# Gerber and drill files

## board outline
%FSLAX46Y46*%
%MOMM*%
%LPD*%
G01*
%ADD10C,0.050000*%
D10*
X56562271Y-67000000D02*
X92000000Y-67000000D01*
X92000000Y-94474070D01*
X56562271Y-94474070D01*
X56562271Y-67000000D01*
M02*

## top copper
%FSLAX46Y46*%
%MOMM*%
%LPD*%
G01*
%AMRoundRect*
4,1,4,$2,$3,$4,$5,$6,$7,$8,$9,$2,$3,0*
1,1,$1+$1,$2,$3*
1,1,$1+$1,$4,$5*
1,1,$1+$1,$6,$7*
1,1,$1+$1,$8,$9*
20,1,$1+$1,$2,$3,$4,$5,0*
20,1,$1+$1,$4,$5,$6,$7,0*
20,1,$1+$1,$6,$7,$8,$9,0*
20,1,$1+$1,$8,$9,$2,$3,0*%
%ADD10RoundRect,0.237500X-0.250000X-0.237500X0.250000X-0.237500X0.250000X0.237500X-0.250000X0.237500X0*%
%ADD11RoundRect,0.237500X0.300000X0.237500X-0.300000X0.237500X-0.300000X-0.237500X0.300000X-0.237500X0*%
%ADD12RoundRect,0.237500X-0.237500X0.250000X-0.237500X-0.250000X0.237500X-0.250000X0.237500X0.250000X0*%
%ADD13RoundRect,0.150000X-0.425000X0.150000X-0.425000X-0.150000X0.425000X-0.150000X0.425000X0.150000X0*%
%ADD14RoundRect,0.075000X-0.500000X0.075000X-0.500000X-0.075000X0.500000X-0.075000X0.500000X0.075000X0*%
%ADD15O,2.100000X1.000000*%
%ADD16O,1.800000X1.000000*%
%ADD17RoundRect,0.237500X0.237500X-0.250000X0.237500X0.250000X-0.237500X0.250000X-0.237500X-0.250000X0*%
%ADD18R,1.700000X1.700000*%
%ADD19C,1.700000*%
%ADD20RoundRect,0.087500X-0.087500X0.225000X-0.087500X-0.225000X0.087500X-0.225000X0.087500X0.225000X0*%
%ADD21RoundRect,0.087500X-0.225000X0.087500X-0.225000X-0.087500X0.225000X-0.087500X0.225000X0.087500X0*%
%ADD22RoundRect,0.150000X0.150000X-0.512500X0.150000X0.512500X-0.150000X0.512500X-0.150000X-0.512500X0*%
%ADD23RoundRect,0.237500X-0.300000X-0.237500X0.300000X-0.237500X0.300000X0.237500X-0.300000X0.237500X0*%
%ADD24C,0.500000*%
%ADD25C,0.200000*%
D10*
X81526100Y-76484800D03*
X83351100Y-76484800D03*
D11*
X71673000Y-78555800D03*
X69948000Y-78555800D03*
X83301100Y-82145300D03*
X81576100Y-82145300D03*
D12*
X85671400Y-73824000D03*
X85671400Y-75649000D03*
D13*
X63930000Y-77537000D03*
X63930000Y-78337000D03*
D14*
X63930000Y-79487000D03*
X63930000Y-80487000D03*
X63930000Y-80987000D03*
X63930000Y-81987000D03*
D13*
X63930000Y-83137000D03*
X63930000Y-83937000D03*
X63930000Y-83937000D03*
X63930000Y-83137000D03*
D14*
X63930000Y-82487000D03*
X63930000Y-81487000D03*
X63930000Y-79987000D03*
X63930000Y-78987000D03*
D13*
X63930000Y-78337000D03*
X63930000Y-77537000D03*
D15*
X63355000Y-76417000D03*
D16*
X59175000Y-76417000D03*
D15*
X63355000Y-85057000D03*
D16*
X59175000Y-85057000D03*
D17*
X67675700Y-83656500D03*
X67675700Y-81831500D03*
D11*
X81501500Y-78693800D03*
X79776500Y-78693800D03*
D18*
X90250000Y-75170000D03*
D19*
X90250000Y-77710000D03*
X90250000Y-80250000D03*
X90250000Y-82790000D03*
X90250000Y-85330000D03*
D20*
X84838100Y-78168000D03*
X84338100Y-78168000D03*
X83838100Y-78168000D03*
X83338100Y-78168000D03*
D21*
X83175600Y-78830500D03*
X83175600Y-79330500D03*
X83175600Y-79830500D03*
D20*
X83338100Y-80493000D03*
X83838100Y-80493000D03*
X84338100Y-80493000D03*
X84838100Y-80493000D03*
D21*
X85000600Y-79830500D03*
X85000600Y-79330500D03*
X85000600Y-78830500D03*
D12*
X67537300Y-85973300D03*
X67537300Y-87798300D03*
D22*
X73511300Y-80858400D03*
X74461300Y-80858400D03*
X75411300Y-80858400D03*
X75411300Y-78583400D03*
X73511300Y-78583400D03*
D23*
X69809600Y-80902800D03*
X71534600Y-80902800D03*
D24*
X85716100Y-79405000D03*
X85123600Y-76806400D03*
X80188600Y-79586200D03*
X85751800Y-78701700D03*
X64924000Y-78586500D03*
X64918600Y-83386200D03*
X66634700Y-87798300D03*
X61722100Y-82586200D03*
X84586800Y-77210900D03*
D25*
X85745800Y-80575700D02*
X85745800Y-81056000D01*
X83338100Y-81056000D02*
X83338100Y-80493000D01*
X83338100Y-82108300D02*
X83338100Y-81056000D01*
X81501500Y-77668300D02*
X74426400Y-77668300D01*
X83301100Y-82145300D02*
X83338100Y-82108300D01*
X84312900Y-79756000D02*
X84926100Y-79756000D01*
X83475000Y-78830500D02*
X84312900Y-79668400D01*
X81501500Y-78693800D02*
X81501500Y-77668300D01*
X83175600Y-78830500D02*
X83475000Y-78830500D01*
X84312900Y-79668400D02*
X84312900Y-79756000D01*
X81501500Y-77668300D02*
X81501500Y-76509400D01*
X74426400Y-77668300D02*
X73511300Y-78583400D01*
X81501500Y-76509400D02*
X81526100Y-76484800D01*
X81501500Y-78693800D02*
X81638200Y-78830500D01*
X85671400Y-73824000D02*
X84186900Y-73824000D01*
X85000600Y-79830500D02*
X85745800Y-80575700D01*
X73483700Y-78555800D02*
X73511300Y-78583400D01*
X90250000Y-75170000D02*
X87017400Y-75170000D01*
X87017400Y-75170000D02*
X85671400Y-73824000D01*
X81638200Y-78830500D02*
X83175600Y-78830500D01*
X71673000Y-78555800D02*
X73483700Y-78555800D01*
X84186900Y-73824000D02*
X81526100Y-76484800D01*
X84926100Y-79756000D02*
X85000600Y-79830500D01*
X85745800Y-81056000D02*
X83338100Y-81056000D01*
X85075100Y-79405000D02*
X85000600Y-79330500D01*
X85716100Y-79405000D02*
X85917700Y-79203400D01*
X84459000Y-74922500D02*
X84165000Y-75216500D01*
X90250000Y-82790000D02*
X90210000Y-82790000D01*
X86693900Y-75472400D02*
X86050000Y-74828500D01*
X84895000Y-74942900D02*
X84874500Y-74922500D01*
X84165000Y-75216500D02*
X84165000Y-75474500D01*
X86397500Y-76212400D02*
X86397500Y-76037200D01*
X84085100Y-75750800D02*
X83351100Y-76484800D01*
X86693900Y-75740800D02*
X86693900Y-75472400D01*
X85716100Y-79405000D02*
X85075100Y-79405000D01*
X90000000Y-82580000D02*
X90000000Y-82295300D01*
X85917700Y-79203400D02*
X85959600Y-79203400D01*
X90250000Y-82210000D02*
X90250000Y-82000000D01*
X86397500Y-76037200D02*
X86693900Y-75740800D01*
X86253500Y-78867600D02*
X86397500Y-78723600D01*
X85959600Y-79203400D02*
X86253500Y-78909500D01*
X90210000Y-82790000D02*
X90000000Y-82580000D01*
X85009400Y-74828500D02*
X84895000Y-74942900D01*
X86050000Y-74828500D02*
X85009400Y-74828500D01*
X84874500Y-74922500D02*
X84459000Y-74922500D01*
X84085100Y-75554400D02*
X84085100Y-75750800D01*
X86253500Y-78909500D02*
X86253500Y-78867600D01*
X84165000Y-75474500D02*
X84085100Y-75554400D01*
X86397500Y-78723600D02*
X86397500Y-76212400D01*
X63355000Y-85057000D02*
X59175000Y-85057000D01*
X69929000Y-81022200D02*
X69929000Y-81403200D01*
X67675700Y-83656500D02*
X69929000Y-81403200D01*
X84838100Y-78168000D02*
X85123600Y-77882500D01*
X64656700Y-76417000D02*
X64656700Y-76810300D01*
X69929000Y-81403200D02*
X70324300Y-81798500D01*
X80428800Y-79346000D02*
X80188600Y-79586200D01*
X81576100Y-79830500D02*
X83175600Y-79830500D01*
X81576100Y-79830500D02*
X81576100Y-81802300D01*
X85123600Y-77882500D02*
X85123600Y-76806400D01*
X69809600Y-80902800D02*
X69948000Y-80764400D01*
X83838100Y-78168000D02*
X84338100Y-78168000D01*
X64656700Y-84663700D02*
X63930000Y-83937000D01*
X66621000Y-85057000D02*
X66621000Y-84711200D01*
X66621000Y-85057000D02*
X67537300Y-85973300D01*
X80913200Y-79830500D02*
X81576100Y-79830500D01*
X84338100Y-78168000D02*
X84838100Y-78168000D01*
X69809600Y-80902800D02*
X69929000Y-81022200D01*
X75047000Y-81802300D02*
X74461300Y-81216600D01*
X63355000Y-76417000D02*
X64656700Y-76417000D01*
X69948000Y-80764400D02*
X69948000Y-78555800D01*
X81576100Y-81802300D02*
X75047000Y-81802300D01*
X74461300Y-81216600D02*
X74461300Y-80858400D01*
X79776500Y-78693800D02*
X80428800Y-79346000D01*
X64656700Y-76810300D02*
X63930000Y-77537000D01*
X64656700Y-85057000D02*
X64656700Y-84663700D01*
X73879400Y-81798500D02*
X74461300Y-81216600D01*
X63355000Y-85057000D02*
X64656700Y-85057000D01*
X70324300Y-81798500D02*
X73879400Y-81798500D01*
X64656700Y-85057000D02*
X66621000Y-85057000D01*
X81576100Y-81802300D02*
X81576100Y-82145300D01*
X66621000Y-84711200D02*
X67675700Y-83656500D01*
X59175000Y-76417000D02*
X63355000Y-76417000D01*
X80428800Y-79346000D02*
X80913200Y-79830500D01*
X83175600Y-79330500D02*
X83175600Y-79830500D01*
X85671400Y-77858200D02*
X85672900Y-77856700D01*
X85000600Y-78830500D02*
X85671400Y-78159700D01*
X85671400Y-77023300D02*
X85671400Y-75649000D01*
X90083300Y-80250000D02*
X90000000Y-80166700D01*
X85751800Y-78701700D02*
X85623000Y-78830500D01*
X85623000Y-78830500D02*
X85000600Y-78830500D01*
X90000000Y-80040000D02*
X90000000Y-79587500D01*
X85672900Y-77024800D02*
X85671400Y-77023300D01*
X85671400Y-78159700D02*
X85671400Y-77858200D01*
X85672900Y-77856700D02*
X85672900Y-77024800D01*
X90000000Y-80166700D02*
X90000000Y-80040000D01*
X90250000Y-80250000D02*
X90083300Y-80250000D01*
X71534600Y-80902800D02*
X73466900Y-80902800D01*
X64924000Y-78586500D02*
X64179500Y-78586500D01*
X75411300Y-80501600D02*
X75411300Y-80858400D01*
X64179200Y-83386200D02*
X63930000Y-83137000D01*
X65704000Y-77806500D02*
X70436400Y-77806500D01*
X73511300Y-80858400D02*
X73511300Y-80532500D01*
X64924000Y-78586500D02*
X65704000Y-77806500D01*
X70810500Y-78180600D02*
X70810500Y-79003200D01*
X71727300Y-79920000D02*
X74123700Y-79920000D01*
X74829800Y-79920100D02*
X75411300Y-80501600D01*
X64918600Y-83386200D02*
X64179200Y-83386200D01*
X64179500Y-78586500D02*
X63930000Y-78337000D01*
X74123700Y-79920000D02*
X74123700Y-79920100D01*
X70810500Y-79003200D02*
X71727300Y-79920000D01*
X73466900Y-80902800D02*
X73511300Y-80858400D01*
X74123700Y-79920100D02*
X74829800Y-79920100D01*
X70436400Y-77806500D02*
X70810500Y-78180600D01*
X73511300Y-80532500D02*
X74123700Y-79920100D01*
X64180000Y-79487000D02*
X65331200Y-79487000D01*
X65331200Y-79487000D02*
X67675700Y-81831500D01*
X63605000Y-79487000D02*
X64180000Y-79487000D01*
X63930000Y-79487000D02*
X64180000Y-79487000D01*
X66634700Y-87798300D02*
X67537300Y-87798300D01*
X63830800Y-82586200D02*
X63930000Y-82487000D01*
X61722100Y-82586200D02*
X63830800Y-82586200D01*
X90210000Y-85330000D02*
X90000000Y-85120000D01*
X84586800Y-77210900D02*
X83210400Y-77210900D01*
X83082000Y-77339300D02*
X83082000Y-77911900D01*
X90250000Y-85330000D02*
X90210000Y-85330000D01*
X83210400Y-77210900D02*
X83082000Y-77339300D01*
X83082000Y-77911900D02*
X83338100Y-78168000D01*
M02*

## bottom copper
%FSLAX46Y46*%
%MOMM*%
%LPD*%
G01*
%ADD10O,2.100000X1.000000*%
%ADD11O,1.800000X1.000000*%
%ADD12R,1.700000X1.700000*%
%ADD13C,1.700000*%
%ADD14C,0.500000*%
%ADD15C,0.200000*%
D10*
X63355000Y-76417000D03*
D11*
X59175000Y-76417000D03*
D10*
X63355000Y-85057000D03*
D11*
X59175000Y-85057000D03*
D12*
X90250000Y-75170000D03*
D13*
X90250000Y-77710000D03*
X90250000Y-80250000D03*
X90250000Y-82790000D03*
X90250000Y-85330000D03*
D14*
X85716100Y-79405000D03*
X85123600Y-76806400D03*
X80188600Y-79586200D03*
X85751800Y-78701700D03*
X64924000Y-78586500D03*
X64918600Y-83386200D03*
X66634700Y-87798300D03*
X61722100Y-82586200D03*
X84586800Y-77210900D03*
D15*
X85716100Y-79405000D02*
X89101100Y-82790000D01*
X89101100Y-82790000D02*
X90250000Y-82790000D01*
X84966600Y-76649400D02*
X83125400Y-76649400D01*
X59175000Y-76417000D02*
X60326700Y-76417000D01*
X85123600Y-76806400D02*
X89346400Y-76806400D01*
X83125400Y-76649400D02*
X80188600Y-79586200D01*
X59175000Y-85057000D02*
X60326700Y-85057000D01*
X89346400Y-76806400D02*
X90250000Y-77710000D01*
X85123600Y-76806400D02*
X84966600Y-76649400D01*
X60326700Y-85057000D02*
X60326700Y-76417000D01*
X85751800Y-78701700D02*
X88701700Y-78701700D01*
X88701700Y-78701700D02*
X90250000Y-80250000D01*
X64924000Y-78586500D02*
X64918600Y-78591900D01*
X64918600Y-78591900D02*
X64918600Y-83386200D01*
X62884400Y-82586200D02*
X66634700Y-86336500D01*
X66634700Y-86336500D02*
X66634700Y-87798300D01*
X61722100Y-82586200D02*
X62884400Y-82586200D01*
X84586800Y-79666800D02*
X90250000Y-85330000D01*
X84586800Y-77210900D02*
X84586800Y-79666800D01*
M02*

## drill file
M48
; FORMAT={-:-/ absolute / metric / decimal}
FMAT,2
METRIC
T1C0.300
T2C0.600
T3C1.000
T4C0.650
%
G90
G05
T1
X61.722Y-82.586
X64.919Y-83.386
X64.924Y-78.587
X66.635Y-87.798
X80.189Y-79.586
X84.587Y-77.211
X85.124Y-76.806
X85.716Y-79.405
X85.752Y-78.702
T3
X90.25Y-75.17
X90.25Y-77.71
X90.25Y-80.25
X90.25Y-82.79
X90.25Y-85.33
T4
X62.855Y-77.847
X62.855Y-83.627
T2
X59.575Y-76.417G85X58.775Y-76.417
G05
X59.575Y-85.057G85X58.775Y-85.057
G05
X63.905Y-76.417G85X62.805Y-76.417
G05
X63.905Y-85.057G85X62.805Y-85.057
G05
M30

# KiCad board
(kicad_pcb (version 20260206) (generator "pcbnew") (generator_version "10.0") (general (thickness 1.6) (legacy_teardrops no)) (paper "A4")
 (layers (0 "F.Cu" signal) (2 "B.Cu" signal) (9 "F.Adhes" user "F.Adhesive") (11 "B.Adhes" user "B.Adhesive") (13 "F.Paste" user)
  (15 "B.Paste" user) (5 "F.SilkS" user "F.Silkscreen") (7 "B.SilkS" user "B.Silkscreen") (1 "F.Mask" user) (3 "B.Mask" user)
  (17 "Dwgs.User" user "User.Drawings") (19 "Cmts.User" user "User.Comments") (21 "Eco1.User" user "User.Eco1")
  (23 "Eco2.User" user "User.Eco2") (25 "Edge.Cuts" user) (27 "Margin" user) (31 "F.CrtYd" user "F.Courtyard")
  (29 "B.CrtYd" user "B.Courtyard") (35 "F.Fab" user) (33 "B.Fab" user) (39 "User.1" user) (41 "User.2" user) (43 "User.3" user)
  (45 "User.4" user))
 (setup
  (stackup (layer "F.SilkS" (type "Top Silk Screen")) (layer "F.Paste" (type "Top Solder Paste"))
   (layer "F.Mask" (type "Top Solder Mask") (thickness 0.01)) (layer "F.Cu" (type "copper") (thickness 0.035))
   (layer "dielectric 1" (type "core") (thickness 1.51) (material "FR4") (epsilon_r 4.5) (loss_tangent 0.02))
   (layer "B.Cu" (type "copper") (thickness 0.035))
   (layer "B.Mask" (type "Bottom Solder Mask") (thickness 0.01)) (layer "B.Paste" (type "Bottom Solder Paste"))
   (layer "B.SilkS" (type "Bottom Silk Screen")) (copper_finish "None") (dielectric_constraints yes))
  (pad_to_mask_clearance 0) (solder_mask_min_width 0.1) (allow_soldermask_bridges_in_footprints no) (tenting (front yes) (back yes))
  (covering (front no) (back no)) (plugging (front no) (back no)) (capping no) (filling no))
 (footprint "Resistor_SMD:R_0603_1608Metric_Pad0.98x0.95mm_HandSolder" (layer "F.Cu") (at 82.4386 76.4848)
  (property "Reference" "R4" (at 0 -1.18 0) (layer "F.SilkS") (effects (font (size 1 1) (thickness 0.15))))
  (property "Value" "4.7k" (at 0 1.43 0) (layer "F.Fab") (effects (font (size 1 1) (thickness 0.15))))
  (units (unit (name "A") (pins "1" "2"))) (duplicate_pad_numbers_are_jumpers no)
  (pad "1" smd roundrect (at -0.9125 0) (size 0.975 0.95) (layers "F.Cu" "F.Mask" "F.Paste") (roundrect_rratio 0.25) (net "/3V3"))
  (pad "2" smd roundrect (at 0.9125 0) (size 0.975 0.95) (layers "F.Cu" "F.Mask" "F.Paste") (roundrect_rratio 0.25) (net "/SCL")))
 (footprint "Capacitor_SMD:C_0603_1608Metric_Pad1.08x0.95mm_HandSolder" (layer "F.Cu") (at 70.8105 78.5558 180)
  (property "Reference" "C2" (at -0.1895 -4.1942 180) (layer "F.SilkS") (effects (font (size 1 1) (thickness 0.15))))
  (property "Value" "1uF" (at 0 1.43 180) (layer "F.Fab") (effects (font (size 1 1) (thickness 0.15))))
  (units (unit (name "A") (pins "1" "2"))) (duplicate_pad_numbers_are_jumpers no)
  (pad "1" smd roundrect (at -0.8625 0 180) (size 1.075 0.95) (layers "F.Cu" "F.Mask" "F.Paste") (roundrect_rratio 0.25) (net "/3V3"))
  (pad "2" smd roundrect (at 0.8625 0 180) (size 1.075 0.95) (layers "F.Cu" "F.Mask" "F.Paste") (roundrect_rratio 0.25) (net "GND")))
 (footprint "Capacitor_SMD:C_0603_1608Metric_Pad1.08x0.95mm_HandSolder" (layer "F.Cu") (at 82.4386 82.1453 180)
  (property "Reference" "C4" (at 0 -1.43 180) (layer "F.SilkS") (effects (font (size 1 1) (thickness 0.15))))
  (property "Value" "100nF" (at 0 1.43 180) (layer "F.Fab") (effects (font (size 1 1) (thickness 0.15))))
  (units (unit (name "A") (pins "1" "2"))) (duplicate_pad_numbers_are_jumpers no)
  (pad "1" smd roundrect (at -0.8625 0 180) (size 1.075 0.95) (layers "F.Cu" "F.Mask" "F.Paste") (roundrect_rratio 0.25) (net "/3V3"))
  (pad "2" smd roundrect (at 0.8625 0 180) (size 1.075 0.95) (layers "F.Cu" "F.Mask" "F.Paste") (roundrect_rratio 0.25) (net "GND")))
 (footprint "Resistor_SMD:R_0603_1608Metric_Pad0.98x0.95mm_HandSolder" (layer "F.Cu") (at 85.6714 74.7365 -90)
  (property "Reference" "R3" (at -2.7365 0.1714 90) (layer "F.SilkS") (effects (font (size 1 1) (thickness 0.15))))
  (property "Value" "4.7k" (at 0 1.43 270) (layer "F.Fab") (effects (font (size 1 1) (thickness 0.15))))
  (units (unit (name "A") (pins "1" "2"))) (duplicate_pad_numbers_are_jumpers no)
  (pad "1" smd roundrect (at -0.9125 0 270) (size 0.975 0.95) (layers "F.Cu" "F.Mask" "F.Paste") (roundrect_rratio 0.25) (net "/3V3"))
  (pad "2" smd roundrect (at 0.9125 0 270) (size 0.975 0.95) (layers "F.Cu" "F.Mask" "F.Paste") (roundrect_rratio 0.25) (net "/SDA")))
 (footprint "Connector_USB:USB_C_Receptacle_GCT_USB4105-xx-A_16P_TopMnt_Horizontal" (layer "F.Cu") (at 60.25 80.737 -90)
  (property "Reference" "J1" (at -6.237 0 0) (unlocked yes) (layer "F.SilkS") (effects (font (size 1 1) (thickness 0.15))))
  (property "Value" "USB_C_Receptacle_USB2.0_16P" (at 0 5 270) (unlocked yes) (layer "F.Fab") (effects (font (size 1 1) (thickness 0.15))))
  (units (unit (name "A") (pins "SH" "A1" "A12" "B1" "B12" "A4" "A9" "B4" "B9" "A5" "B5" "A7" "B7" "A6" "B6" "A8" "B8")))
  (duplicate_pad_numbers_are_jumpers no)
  (pad "" np_thru_hole circle (at -2.89 -2.605 270) (size 0.65 0.65) (drill 0.65) (layers "*.Cu" "*.Mask"))
  (pad "" np_thru_hole circle (at 2.89 -2.605 270) (size 0.65 0.65) (drill 0.65) (layers "*.Cu" "*.Mask"))
  (pad "A1" smd roundrect (at -3.2 -3.68 270) (size 0.6 1.15) (layers "F.Cu" "F.Mask" "F.Paste") (roundrect_rratio 0.25) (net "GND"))
  (pad "A4" smd roundrect (at -2.4 -3.68 270) (size 0.6 1.15) (layers "F.Cu" "F.Mask" "F.Paste") (roundrect_rratio 0.25) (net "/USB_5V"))
  (pad "A5" smd roundrect (at -1.25 -3.68 270) (size 0.3 1.15) (layers "F.Cu" "F.Mask" "F.Paste") (roundrect_rratio 0.25)
   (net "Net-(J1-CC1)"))
  (pad "A6" smd roundrect (at -0.25 -3.68 270) (size 0.3 1.15) (layers "F.Cu" "F.Mask" "F.Paste") (roundrect_rratio 0.25)
   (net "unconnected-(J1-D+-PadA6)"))
  (pad "A7" smd roundrect (at 0.25 -3.68 270) (size 0.3 1.15) (layers "F.Cu" "F.Mask" "F.Paste") (roundrect_rratio 0.25)
   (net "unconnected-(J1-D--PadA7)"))
  (pad "A8" smd roundrect (at 1.25 -3.68 270) (size 0.3 1.15) (layers "F.Cu" "F.Mask" "F.Paste") (roundrect_rratio 0.25)
   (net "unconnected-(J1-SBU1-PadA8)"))
  (pad "A9" smd roundrect (at 2.4 -3.68 270) (size 0.6 1.15) (layers "F.Cu" "F.Mask" "F.Paste") (roundrect_rratio 0.25) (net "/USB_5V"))
  (pad "A12" smd roundrect (at 3.2 -3.68 270) (size 0.6 1.15) (layers "F.Cu" "F.Mask" "F.Paste") (roundrect_rratio 0.25) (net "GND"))
  (pad "B1" smd roundrect (at 3.2 -3.68 270) (size 0.6 1.15) (layers "F.Cu" "F.Mask" "F.Paste") (roundrect_rratio 0.25) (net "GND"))
  (pad "B4" smd roundrect (at 2.4 -3.68 270) (size 0.6 1.15) (layers "F.Cu" "F.Mask" "F.Paste") (roundrect_rratio 0.25) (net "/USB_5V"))
  (pad "B5" smd roundrect (at 1.75 -3.68 270) (size 0.3 1.15) (layers "F.Cu" "F.Mask" "F.Paste") (roundrect_rratio 0.25)
   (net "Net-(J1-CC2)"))
  (pad "B6" smd roundrect (at 0.75 -3.68 270) (size 0.3 1.15) (layers "F.Cu" "F.Mask" "F.Paste") (roundrect_rratio 0.25)
   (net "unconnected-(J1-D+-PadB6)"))
  (pad "B7" smd roundrect (at -0.75 -3.68 270) (size 0.3 1.15) (layers "F.Cu" "F.Mask" "F.Paste") (roundrect_rratio 0.25)
   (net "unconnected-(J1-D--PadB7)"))
  (pad "B8" smd roundrect (at -1.75 -3.68 270) (size 0.3 1.15) (layers "F.Cu" "F.Mask" "F.Paste") (roundrect_rratio 0.25)
   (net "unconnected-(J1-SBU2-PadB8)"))
  (pad "B9" smd roundrect (at -2.4 -3.68 270) (size 0.6 1.15) (layers "F.Cu" "F.Mask" "F.Paste") (roundrect_rratio 0.25) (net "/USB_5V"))
  (pad "B12" smd roundrect (at -3.2 -3.68 270) (size 0.6 1.15) (layers "F.Cu" "F.Mask" "F.Paste") (roundrect_rratio 0.25) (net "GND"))
  (pad "SH" thru_hole oval (at -4.32 -3.105 270) (size 1 2.1) (drill oval 0.6 1.7) (layers "*.Cu" "*.Mask" "F.Paste")
   (remove_unused_layers no) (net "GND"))
  (pad "SH" thru_hole oval (at -4.32 1.075 270) (size 1 1.8) (drill oval 0.6 1.4) (layers "*.Cu" "*.Mask" "F.Paste")
   (remove_unused_layers no) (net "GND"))
  (pad "SH" thru_hole oval (at 4.32 -3.105 270) (size 1 2.1) (drill oval 0.6 1.7) (layers "*.Cu" "*.Mask" "F.Paste")
   (remove_unused_layers no) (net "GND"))
  (pad "SH" thru_hole oval (at 4.32 1.075 270) (size 1 1.8) (drill oval 0.6 1.4) (layers "*.Cu" "*.Mask" "F.Paste")
   (remove_unused_layers no) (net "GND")))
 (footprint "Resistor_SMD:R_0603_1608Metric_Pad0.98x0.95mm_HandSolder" (layer "F.Cu") (at 67.6757 82.744 90)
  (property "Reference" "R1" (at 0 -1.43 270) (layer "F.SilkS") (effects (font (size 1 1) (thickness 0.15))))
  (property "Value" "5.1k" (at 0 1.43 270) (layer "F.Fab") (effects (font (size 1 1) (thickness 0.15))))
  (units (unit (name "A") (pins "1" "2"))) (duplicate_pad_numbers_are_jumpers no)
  (pad "1" smd roundrect (at -0.9125 0 90) (size 0.975 0.95) (layers "F.Cu" "F.Mask" "F.Paste") (roundrect_rratio 0.25) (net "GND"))
  (pad "2" smd roundrect (at 0.9125 0 90) (size 0.975 0.95) (layers "F.Cu" "F.Mask" "F.Paste") (roundrect_rratio 0.25) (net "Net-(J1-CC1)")))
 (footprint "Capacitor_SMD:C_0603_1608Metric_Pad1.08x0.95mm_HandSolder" (layer "F.Cu") (at 80.639 78.6938 180)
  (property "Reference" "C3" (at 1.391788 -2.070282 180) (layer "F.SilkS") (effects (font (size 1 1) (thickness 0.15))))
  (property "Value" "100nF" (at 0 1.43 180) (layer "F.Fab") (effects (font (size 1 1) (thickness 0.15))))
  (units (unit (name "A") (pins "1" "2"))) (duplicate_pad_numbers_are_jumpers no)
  (pad "1" smd roundrect (at -0.8625 0 180) (size 1.075 0.95) (layers "F.Cu" "F.Mask" "F.Paste") (roundrect_rratio 0.25) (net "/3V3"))
  (pad "2" smd roundrect (at 0.8625 0 180) (size 1.075 0.95) (layers "F.Cu" "F.Mask" "F.Paste") (roundrect_rratio 0.25) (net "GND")))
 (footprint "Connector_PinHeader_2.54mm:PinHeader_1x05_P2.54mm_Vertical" (layer "F.Cu") (at 90.25 75.17)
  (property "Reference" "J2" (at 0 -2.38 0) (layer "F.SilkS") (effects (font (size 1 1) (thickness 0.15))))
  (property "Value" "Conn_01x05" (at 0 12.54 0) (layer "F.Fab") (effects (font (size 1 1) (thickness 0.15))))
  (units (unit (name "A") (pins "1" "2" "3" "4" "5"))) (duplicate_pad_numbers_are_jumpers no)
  (pad "1" thru_hole rect (at 0 0) (size 1.7 1.7) (drill 1) (layers "*.Cu" "*.Mask") (remove_unused_layers no) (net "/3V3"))
  (pad "2" thru_hole circle (at 0 2.54) (size 1.7 1.7) (drill 1) (layers "*.Cu" "*.Mask") (remove_unused_layers no) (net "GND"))
  (pad "3" thru_hole circle (at 0 5.08) (size 1.7 1.7) (drill 1) (layers "*.Cu" "*.Mask") (remove_unused_layers no) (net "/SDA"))
  (pad "4" thru_hole circle (at 0 7.62) (size 1.7 1.7) (drill 1) (layers "*.Cu" "*.Mask") (remove_unused_layers no) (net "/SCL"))
  (pad "5" thru_hole circle (at 0 10.16) (size 1.7 1.7) (drill 1) (layers "*.Cu" "*.Mask") (remove_unused_layers no) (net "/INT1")))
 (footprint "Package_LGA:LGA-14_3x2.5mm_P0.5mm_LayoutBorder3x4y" (layer "F.Cu") (at 84.0881 79.3305 -90)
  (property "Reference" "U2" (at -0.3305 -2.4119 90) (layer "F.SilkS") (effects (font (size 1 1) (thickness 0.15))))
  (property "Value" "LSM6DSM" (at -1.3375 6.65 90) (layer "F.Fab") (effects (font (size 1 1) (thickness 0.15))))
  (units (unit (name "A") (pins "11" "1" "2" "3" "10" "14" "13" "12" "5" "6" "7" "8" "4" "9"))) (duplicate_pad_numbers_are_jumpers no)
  (pad "1" smd roundrect (at -1.1625 -0.75 270) (size 0.625 0.35) (layers "F.Cu" "F.Mask" "F.Paste") (roundrect_rratio 0.25) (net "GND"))
  (pad "2" smd roundrect (at -1.1625 -0.25 270) (size 0.625 0.35) (layers "F.Cu" "F.Mask" "F.Paste") (roundrect_rratio 0.25) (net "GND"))
  (pad "3" smd roundrect (at -1.1625 0.25 270) (size 0.625 0.35) (layers "F.Cu" "F.Mask" "F.Paste") (roundrect_rratio 0.25) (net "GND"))
  (pad "4" smd roundrect (at -1.1625 0.75 270) (size 0.625 0.35) (layers "F.Cu" "F.Mask" "F.Paste") (roundrect_rratio 0.25) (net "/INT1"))
  (pad "5" smd roundrect (at -0.5 0.9125 270) (size 0.35 0.625) (layers "F.Cu" "F.Mask" "F.Paste") (roundrect_rratio 0.25) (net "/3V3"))
  (pad "6" smd roundrect (at 0 0.9125 270) (size 0.35 0.625) (layers "F.Cu" "F.Mask" "F.Paste") (roundrect_rratio 0.25) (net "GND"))
  (pad "7" smd roundrect (at 0.5 0.9125 270) (size 0.35 0.625) (layers "F.Cu" "F.Mask" "F.Paste") (roundrect_rratio 0.25) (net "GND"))
  (pad "8" smd roundrect (at 1.1625 0.75 270) (size 0.625 0.35) (layers "F.Cu" "F.Mask" "F.Paste") (roundrect_rratio 0.25) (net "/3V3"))
  (pad "9" smd roundrect (at 1.1625 0.25 270) (size 0.625 0.35) (layers "F.Cu" "F.Mask" "F.Paste") (roundrect_rratio 0.25)
   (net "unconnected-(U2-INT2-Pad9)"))
  (pad "10" smd roundrect (at 1.1625 -0.25 270) (size 0.625 0.35) (layers "F.Cu" "F.Mask" "F.Paste") (roundrect_rratio 0.25)
   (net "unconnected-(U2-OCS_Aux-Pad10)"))
  (pad "11" smd roundrect (at 1.1625 -0.75 270) (size 0.625 0.35) (layers "F.Cu" "F.Mask" "F.Paste") (roundrect_rratio 0.25)
   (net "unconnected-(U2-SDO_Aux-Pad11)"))
  (pad "12" smd roundrect (at 0.5 -0.9125 270) (size 0.35 0.625) (layers "F.Cu" "F.Mask" "F.Paste") (roundrect_rratio 0.25) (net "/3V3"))
  (pad "13" smd roundrect (at 0 -0.9125 270) (size 0.35 0.625) (layers "F.Cu" "F.Mask" "F.Paste") (roundrect_rratio 0.25) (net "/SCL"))
  (pad "14" smd roundrect (at -0.5 -0.9125 270) (size 0.35 0.625) (layers "F.Cu" "F.Mask" "F.Paste") (roundrect_rratio 0.25) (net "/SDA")))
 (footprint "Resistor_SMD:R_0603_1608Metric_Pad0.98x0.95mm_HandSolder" (layer "F.Cu") (at 67.5373 86.8858 -90)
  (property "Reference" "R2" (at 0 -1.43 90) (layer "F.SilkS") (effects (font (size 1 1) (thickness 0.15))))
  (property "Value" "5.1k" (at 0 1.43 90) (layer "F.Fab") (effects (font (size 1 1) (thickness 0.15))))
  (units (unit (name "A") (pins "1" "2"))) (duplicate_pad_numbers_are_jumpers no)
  (pad "1" smd roundrect (at -0.9125 0 270) (size 0.975 0.95) (layers "F.Cu" "F.Mask" "F.Paste") (roundrect_rratio 0.25) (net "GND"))
  (pad "2" smd roundrect (at 0.9125 0 270) (size 0.975 0.95) (layers "F.Cu" "F.Mask" "F.Paste") (roundrect_rratio 0.25) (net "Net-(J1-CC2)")))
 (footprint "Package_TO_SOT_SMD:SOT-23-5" (layer "F.Cu") (at 74.4613 79.7209 90)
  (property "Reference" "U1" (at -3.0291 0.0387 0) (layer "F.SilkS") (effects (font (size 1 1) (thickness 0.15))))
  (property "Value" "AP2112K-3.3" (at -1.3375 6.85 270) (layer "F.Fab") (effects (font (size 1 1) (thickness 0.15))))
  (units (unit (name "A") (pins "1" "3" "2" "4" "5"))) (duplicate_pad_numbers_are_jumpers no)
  (pad "1" smd roundrect (at -1.1375 -0.95 90) (size 1.325 0.6) (layers "F.Cu" "F.Mask" "F.Paste") (roundrect_rratio 0.25) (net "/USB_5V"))
  (pad "2" smd roundrect (at -1.1375 0 90) (size 1.325 0.6) (layers "F.Cu" "F.Mask" "F.Paste") (roundrect_rratio 0.25) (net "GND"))
  (pad "3" smd roundrect (at -1.1375 0.95 90) (size 1.325 0.6) (layers "F.Cu" "F.Mask" "F.Paste") (roundrect_rratio 0.25) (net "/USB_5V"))
  (pad "4" smd roundrect (at 1.1375 0.95 90) (size 1.325 0.6) (layers "F.Cu" "F.Mask" "F.Paste") (roundrect_rratio 0.25)
   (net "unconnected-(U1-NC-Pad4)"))
  (pad "5" smd roundrect (at 1.1375 -0.95 90) (size 1.325 0.6) (layers "F.Cu" "F.Mask" "F.Paste") (roundrect_rratio 0.25) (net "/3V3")))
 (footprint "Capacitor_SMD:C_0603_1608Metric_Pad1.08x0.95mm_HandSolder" (layer "F.Cu") (at 70.6721 80.9028)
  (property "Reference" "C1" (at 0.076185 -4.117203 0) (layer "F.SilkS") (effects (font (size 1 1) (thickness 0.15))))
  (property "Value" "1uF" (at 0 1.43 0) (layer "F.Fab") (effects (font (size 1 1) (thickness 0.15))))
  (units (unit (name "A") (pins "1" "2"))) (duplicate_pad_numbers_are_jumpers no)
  (pad "1" smd roundrect (at -0.8625 0) (size 1.075 0.95) (layers "F.Cu" "F.Mask" "F.Paste") (roundrect_rratio 0.25) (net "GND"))
  (pad "2" smd roundrect (at 0.8625 0) (size 1.075 0.95) (layers "F.Cu" "F.Mask" "F.Paste") (roundrect_rratio 0.25) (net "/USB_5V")))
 (gr_rect (start 56.562271 67) (end 92 94.47407) (stroke (width 0.05) (type default)) (fill no) (layer "Edge.Cuts"))
 (segment (start 85.7458 80.5757) (end 85.7458 81.056) (width 0.2) (layer "F.Cu") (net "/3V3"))
 (segment (start 83.3381 81.056) (end 83.3381 80.493) (width 0.2) (layer "F.Cu") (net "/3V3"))
 (segment (start 83.3381 82.1083) (end 83.3381 81.056) (width 0.2) (layer "F.Cu") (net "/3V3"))
 (segment (start 81.5015 77.6683) (end 74.4264 77.6683) (width 0.2) (layer "F.Cu") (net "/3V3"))
 (segment (start 83.3011 82.1453) (end 83.3381 82.1083) (width 0.2) (layer "F.Cu") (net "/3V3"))
 (segment (start 84.3129 79.756) (end 84.9261 79.756) (width 0.2) (layer "F.Cu") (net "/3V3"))
 (segment (start 83.475 78.8305) (end 84.3129 79.6684) (width 0.2) (layer "F.Cu") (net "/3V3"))
 (segment (start 81.5015 78.6938) (end 81.5015 77.6683) (width 0.2) (layer "F.Cu") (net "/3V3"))
 (segment (start 83.1756 78.8305) (end 83.475 78.8305) (width 0.2) (layer "F.Cu") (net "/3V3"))
 (segment (start 84.3129 79.6684) (end 84.3129 79.756) (width 0.2) (layer "F.Cu") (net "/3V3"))
 (segment (start 81.5015 77.6683) (end 81.5015 76.5094) (width 0.2) (layer "F.Cu") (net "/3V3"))
 (segment (start 74.4264 77.6683) (end 73.5113 78.5834) (width 0.2) (layer "F.Cu") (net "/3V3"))
 (segment (start 81.5015 76.5094) (end 81.5261 76.4848) (width 0.2) (layer "F.Cu") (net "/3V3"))
 (segment (start 81.5015 78.6938) (end 81.6382 78.8305) (width 0.2) (layer "F.Cu") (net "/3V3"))
 (segment (start 85.6714 73.824) (end 84.1869 73.824) (width 0.2) (layer "F.Cu") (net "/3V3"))
 (segment (start 85.0006 79.8305) (end 85.7458 80.5757) (width 0.2) (layer "F.Cu") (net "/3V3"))
 (segment (start 73.4837 78.5558) (end 73.5113 78.5834) (width 0.2) (layer "F.Cu") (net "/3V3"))
 (segment (start 90.25 75.17) (end 87.0174 75.17) (width 0.2) (layer "F.Cu") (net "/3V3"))
 (segment (start 87.0174 75.17) (end 85.6714 73.824) (width 0.2) (layer "F.Cu") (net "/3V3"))
 (segment (start 81.6382 78.8305) (end 83.1756 78.8305) (width 0.2) (layer "F.Cu") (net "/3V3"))
 (segment (start 71.673 78.5558) (end 73.4837 78.5558) (width 0.2) (layer "F.Cu") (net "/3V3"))
 (segment (start 84.1869 73.824) (end 81.5261 76.4848) (width 0.2) (layer "F.Cu") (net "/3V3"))
 (segment (start 84.9261 79.756) (end 85.0006 79.8305) (width 0.2) (layer "F.Cu") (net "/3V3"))
 (segment (start 85.7458 81.056) (end 83.3381 81.056) (width 0.2) (layer "F.Cu") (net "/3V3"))
 (segment (start 85.0751 79.405) (end 85.0006 79.3305) (width 0.2) (layer "F.Cu") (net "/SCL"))
 (segment (start 85.7161 79.405) (end 85.9177 79.2034) (width 0.2) (layer "F.Cu") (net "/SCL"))
 (segment (start 84.459 74.9225) (end 84.165 75.2165) (width 0.2) (layer "F.Cu") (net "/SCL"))
 (segment (start 90.25 82.79) (end 90.21 82.79) (width 0.2) (layer "F.Cu") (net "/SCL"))
 (segment (start 86.6939 75.4724) (end 86.05 74.8285) (width 0.2) (layer "F.Cu") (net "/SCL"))
 (segment (start 84.895 74.9429) (end 84.8745 74.9225) (width 0.2) (layer "F.Cu") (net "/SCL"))
 (segment (start 84.165 75.2165) (end 84.165 75.4745) (width 0.2) (layer "F.Cu") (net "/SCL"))
 (segment (start 86.3975 76.2124) (end 86.3975 76.0372) (width 0.2) (layer "F.Cu") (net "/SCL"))
 (segment (start 84.0851 75.7508) (end 83.3511 76.4848) (width 0.2) (layer "F.Cu") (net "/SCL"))
 (segment (start 86.6939 75.7408) (end 86.6939 75.4724) (width 0.2) (layer "F.Cu") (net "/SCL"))
 (segment (start 85.7161 79.405) (end 85.0751 79.405) (width 0.2) (layer "F.Cu") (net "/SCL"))
 (segment (start 90 82.58) (end 90 82.2953) (width 0.2) (layer "F.Cu") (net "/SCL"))
 (segment (start 85.9177 79.2034) (end 85.9596 79.2034) (width 0.2) (layer "F.Cu") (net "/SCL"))
 (segment (start 90.25 82.21) (end 90.25 82) (width 0.2) (layer "F.Cu") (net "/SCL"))
 (segment (start 86.3975 76.0372) (end 86.6939 75.7408) (width 0.2) (layer "F.Cu") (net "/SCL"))
 (segment (start 86.2535 78.8676) (end 86.3975 78.7236) (width 0.2) (layer "F.Cu") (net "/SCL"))
 (segment (start 85.9596 79.2034) (end 86.2535 78.9095) (width 0.2) (layer "F.Cu") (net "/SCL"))
 (segment (start 90.21 82.79) (end 90 82.58) (width 0.2) (layer "F.Cu") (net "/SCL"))
 (segment (start 85.0094 74.8285) (end 84.895 74.9429) (width 0.2) (layer "F.Cu") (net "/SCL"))
 (segment (start 86.05 74.8285) (end 85.0094 74.8285) (width 0.2) (layer "F.Cu") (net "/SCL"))
 (segment (start 84.8745 74.9225) (end 84.459 74.9225) (width 0.2) (layer "F.Cu") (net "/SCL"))
 (segment (start 84.0851 75.5544) (end 84.0851 75.7508) (width 0.2) (layer "F.Cu") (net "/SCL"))
 (segment (start 86.2535 78.9095) (end 86.2535 78.8676) (width 0.2) (layer "F.Cu") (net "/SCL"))
 (segment (start 84.165 75.4745) (end 84.0851 75.5544) (width 0.2) (layer "F.Cu") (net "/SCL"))
 (segment (start 86.3975 78.7236) (end 86.3975 76.2124) (width 0.2) (layer "F.Cu") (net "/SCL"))
 (via (at 85.7161 79.405) (size 0.5) (drill 0.3) (layers "F.Cu" "B.Cu") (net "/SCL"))
 (segment (start 85.7161 79.405) (end 89.1011 82.79) (width 0.2) (layer "B.Cu") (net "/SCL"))
 (segment (start 89.1011 82.79) (end 90.25 82.79) (width 0.2) (layer "B.Cu") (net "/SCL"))
 (segment (start 63.355 85.057) (end 59.175 85.057) (width 0.2) (layer "F.Cu") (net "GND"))
 (segment (start 69.929 81.0222) (end 69.929 81.4032) (width 0.2) (layer "F.Cu") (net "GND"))
 (segment (start 67.6757 83.6565) (end 69.929 81.4032) (width 0.2) (layer "F.Cu") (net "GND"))
 (segment (start 84.8381 78.168) (end 85.1236 77.8825) (width 0.2) (layer "F.Cu") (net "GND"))
 (segment (start 64.6567 76.417) (end 64.6567 76.8103) (width 0.2) (layer "F.Cu") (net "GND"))
 (segment (start 69.929 81.4032) (end 70.3243 81.7985) (width 0.2) (layer "F.Cu") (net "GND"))
 (segment (start 80.4288 79.346) (end 80.1886 79.5862) (width 0.2) (layer "F.Cu") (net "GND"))
 (segment (start 81.5761 79.8305) (end 83.1756 79.8305) (width 0.2) (layer "F.Cu") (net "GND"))
 (segment (start 81.5761 79.8305) (end 81.5761 81.8023) (width 0.2) (layer "F.Cu") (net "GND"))
 (segment (start 85.1236 77.8825) (end 85.1236 76.8064) (width 0.2) (layer "F.Cu") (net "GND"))
 (segment (start 69.8096 80.9028) (end 69.948 80.7644) (width 0.2) (layer "F.Cu") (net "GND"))
 (segment (start 83.8381 78.168) (end 84.3381 78.168) (width 0.2) (layer "F.Cu") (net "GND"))
 (segment (start 64.6567 84.6637) (end 63.93 83.937) (width 0.2) (layer "F.Cu") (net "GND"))
 (segment (start 66.621 85.057) (end 66.621 84.7112) (width 0.2) (layer "F.Cu") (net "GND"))
 (segment (start 66.621 85.057) (end 67.5373 85.9733) (width 0.2) (layer "F.Cu") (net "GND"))
 (segment (start 80.9132 79.8305) (end 81.5761 79.8305) (width 0.2) (layer "F.Cu") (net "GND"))
 (segment (start 84.3381 78.168) (end 84.8381 78.168) (width 0.2) (layer "F.Cu") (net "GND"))
 (segment (start 69.8096 80.9028) (end 69.929 81.0222) (width 0.2) (layer "F.Cu") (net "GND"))
 (segment (start 75.047 81.8023) (end 74.4613 81.2166) (width 0.2) (layer "F.Cu") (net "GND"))
 (segment (start 63.355 76.417) (end 64.6567 76.417) (width 0.2) (layer "F.Cu") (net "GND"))
 (segment (start 69.948 80.7644) (end 69.948 78.5558) (width 0.2) (layer "F.Cu") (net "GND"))
 (segment (start 81.5761 81.8023) (end 75.047 81.8023) (width 0.2) (layer "F.Cu") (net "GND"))
 (segment (start 74.4613 81.2166) (end 74.4613 80.8584) (width 0.2) (layer "F.Cu") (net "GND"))
 (segment (start 79.7765 78.6938) (end 80.4288 79.346) (width 0.2) (layer "F.Cu") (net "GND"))
 (segment (start 64.6567 76.8103) (end 63.93 77.537) (width 0.2) (layer "F.Cu") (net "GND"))
 (segment (start 64.6567 85.057) (end 64.6567 84.6637) (width 0.2) (layer "F.Cu") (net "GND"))
 (segment (start 73.8794 81.7985) (end 74.4613 81.2166) (width 0.2) (layer "F.Cu") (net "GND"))
 (segment (start 63.355 85.057) (end 64.6567 85.057) (width 0.2) (layer "F.Cu") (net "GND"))
 (segment (start 70.3243 81.7985) (end 73.8794 81.7985) (width 0.2) (layer "F.Cu") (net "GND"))
 (segment (start 64.6567 85.057) (end 66.621 85.057) (width 0.2) (layer "F.Cu") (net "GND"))
 (segment (start 81.5761 81.8023) (end 81.5761 82.1453) (width 0.2) (layer "F.Cu") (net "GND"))
 (segment (start 66.621 84.7112) (end 67.6757 83.6565) (width 0.2) (layer "F.Cu") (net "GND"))
 (segment (start 59.175 76.417) (end 63.355 76.417) (width 0.2) (layer "F.Cu") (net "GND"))
 (segment (start 80.4288 79.346) (end 80.9132 79.8305) (width 0.2) (layer "F.Cu") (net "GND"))
 (segment (start 83.1756 79.3305) (end 83.1756 79.8305) (width 0.2) (layer "F.Cu") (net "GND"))
 (via (at 85.1236 76.8064) (size 0.5) (drill 0.3) (layers "F.Cu" "B.Cu") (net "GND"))
 (via (at 80.1886 79.5862) (size 0.5) (drill 0.3) (layers "F.Cu" "B.Cu") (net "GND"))
 (segment (start 84.9666 76.6494) (end 83.1254 76.6494) (width 0.2) (layer "B.Cu") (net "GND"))
 (segment (start 59.175 76.417) (end 60.3267 76.417) (width 0.2) (layer "B.Cu") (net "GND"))
 (segment (start 85.1236 76.8064) (end 89.3464 76.8064) (width 0.2) (layer "B.Cu") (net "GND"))
 (segment (start 83.1254 76.6494) (end 80.1886 79.5862) (width 0.2) (layer "B.Cu") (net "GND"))
 (segment (start 59.175 85.057) (end 60.3267 85.057) (width 0.2) (layer "B.Cu") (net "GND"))
 (segment (start 89.3464 76.8064) (end 90.25 77.71) (width 0.2) (layer "B.Cu") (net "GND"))
 (segment (start 85.1236 76.8064) (end 84.9666 76.6494) (width 0.2) (layer "B.Cu") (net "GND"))
 (segment (start 60.3267 85.057) (end 60.3267 76.417) (width 0.2) (layer "B.Cu") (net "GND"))
 (segment (start 85.6714 77.8582) (end 85.6729 77.8567) (width 0.2) (layer "F.Cu") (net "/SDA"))
 (segment (start 85.0006 78.8305) (end 85.6714 78.1597) (width 0.2) (layer "F.Cu") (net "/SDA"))
 (segment (start 85.6714 77.0233) (end 85.6714 75.649) (width 0.2) (layer "F.Cu") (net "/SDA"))
 (segment (start 90.0833 80.25) (end 90 80.1667) (width 0.2) (layer "F.Cu") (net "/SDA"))
 (segment (start 85.7518 78.7017) (end 85.623 78.8305) (width 0.2) (layer "F.Cu") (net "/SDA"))
 (segment (start 85.623 78.8305) (end 85.0006 78.8305) (width 0.2) (layer "F.Cu") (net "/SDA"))
 (segment (start 90 80.04) (end 90 79.5875) (width 0.2) (layer "F.Cu") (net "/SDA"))
 (segment (start 85.6729 77.0248) (end 85.6714 77.0233) (width 0.2) (layer "F.Cu") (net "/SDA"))
 (segment (start 85.6714 78.1597) (end 85.6714 77.8582) (width 0.2) (layer "F.Cu") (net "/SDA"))
 (segment (start 85.6729 77.8567) (end 85.6729 77.0248) (width 0.2) (layer "F.Cu") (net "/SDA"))
 (segment (start 90 80.1667) (end 90 80.04) (width 0.2) (layer "F.Cu") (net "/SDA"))
 (segment (start 90.25 80.25) (end 90.0833 80.25) (width 0.2) (layer "F.Cu") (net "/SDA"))
 (via (at 85.7518 78.7017) (size 0.5) (drill 0.3) (layers "F.Cu" "B.Cu") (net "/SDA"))
 (segment (start 85.7518 78.7017) (end 88.7017 78.7017) (width 0.2) (layer "B.Cu") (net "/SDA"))
 (segment (start 88.7017 78.7017) (end 90.25 80.25) (width 0.2) (layer "B.Cu") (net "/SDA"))
 (segment (start 71.5346 80.9028) (end 73.4669 80.9028) (width 0.2) (layer "F.Cu") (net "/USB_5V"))
 (segment (start 64.924 78.5865) (end 64.1795 78.5865) (width 0.2) (layer "F.Cu") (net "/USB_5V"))
 (segment (start 75.4113 80.5016) (end 75.4113 80.8584) (width 0.2) (layer "F.Cu") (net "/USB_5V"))
 (segment (start 64.1792 83.3862) (end 63.93 83.137) (width 0.2) (layer "F.Cu") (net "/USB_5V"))
 (segment (start 65.704 77.8065) (end 70.4364 77.8065) (width 0.2) (layer "F.Cu") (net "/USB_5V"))
 (segment (start 73.5113 80.8584) (end 73.5113 80.5325) (width 0.2) (layer "F.Cu") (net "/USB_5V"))
 (segment (start 64.924 78.5865) (end 65.704 77.8065) (width 0.2) (layer "F.Cu") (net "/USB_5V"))
 (segment (start 70.8105 78.1806) (end 70.8105 79.0032) (width 0.2) (layer "F.Cu") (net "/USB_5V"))
 (segment (start 71.7273 79.92) (end 74.1237 79.92) (width 0.2) (layer "F.Cu") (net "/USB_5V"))
 (segment (start 74.8298 79.9201) (end 75.4113 80.5016) (width 0.2) (layer "F.Cu") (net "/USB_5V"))
 (segment (start 64.9186 83.3862) (end 64.1792 83.3862) (width 0.2) (layer "F.Cu") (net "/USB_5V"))
 (segment (start 64.1795 78.5865) (end 63.93 78.337) (width 0.2) (layer "F.Cu") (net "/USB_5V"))
 (segment (start 74.1237 79.92) (end 74.1237 79.9201) (width 0.2) (layer "F.Cu") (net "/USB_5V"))
 (segment (start 70.8105 79.0032) (end 71.7273 79.92) (width 0.2) (layer "F.Cu") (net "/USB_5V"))
 (segment (start 73.4669 80.9028) (end 73.5113 80.8584) (width 0.2) (layer "F.Cu") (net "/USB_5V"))
 (segment (start 74.1237 79.9201) (end 74.8298 79.9201) (width 0.2) (layer "F.Cu") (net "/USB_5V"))
 (segment (start 70.4364 77.8065) (end 70.8105 78.1806) (width 0.2) (layer "F.Cu") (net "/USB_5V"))
 (segment (start 73.5113 80.5325) (end 74.1237 79.9201) (width 0.2) (layer "F.Cu") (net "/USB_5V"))
 (via (at 64.924 78.5865) (size 0.5) (drill 0.3) (layers "F.Cu" "B.Cu") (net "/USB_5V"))
 (via (at 64.9186 83.3862) (size 0.5) (drill 0.3) (layers "F.Cu" "B.Cu") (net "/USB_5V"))
 (segment (start 64.924 78.5865) (end 64.9186 78.5919) (width 0.2) (layer "B.Cu") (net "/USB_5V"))
 (segment (start 64.9186 78.5919) (end 64.9186 83.3862) (width 0.2) (layer "B.Cu") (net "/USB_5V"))
 (segment (start 64.18 79.487) (end 65.3312 79.487) (width 0.2) (layer "F.Cu") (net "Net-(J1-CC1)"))
 (segment (start 65.3312 79.487) (end 67.6757 81.8315) (width 0.2) (layer "F.Cu") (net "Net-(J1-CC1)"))
 (segment (start 63.605 79.487) (end 64.18 79.487) (width 0.2) (layer "F.Cu") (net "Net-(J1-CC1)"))
 (segment (start 63.93 79.487) (end 64.18 79.487) (width 0.2) (layer "F.Cu") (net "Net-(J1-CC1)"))
 (segment (start 66.6347 87.7983) (end 67.5373 87.7983) (width 0.2) (layer "F.Cu") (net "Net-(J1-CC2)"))
 (segment (start 63.8308 82.5862) (end 63.93 82.487) (width 0.2) (layer "F.Cu") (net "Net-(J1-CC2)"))
 (segment (start 61.7221 82.5862) (end 63.8308 82.5862) (width 0.2) (layer "F.Cu") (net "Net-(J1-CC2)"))
 (via (at 66.6347 87.7983) (size 0.5) (drill 0.3) (layers "F.Cu" "B.Cu") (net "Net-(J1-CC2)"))
 (via (at 61.7221 82.5862) (size 0.5) (drill 0.3) (layers "F.Cu" "B.Cu") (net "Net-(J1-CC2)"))
 (segment (start 62.8844 82.5862) (end 66.6347 86.3365) (width 0.2) (layer "B.Cu") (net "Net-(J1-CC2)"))
 (segment (start 66.6347 86.3365) (end 66.6347 87.7983) (width 0.2) (layer "B.Cu") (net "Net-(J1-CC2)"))
 (segment (start 61.7221 82.5862) (end 62.8844 82.5862) (width 0.2) (layer "B.Cu") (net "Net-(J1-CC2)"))
 (segment (start 90.21 85.33) (end 90 85.12) (width 0.2) (layer "F.Cu") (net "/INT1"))
 (segment (start 84.5868 77.2109) (end 83.2104 77.2109) (width 0.2) (layer "F.Cu") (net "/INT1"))
 (segment (start 83.082 77.3393) (end 83.082 77.9119) (width 0.2) (layer "F.Cu") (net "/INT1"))
 (segment (start 90.25 85.33) (end 90.21 85.33) (width 0.2) (layer "F.Cu") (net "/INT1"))
 (segment (start 83.2104 77.2109) (end 83.082 77.3393) (width 0.2) (layer "F.Cu") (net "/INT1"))
 (segment (start 83.082 77.9119) (end 83.3381 78.168) (width 0.2) (layer "F.Cu") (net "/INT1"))
 (via (at 84.5868 77.2109) (size 0.5) (drill 0.3) (layers "F.Cu" "B.Cu") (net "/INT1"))
 (segment (start 84.5868 79.6668) (end 90.25 85.33) (width 0.2) (layer "B.Cu") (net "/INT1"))
 (segment (start 84.5868 77.2109) (end 84.5868 79.6668) (width 0.2) (layer "B.Cu") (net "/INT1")))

